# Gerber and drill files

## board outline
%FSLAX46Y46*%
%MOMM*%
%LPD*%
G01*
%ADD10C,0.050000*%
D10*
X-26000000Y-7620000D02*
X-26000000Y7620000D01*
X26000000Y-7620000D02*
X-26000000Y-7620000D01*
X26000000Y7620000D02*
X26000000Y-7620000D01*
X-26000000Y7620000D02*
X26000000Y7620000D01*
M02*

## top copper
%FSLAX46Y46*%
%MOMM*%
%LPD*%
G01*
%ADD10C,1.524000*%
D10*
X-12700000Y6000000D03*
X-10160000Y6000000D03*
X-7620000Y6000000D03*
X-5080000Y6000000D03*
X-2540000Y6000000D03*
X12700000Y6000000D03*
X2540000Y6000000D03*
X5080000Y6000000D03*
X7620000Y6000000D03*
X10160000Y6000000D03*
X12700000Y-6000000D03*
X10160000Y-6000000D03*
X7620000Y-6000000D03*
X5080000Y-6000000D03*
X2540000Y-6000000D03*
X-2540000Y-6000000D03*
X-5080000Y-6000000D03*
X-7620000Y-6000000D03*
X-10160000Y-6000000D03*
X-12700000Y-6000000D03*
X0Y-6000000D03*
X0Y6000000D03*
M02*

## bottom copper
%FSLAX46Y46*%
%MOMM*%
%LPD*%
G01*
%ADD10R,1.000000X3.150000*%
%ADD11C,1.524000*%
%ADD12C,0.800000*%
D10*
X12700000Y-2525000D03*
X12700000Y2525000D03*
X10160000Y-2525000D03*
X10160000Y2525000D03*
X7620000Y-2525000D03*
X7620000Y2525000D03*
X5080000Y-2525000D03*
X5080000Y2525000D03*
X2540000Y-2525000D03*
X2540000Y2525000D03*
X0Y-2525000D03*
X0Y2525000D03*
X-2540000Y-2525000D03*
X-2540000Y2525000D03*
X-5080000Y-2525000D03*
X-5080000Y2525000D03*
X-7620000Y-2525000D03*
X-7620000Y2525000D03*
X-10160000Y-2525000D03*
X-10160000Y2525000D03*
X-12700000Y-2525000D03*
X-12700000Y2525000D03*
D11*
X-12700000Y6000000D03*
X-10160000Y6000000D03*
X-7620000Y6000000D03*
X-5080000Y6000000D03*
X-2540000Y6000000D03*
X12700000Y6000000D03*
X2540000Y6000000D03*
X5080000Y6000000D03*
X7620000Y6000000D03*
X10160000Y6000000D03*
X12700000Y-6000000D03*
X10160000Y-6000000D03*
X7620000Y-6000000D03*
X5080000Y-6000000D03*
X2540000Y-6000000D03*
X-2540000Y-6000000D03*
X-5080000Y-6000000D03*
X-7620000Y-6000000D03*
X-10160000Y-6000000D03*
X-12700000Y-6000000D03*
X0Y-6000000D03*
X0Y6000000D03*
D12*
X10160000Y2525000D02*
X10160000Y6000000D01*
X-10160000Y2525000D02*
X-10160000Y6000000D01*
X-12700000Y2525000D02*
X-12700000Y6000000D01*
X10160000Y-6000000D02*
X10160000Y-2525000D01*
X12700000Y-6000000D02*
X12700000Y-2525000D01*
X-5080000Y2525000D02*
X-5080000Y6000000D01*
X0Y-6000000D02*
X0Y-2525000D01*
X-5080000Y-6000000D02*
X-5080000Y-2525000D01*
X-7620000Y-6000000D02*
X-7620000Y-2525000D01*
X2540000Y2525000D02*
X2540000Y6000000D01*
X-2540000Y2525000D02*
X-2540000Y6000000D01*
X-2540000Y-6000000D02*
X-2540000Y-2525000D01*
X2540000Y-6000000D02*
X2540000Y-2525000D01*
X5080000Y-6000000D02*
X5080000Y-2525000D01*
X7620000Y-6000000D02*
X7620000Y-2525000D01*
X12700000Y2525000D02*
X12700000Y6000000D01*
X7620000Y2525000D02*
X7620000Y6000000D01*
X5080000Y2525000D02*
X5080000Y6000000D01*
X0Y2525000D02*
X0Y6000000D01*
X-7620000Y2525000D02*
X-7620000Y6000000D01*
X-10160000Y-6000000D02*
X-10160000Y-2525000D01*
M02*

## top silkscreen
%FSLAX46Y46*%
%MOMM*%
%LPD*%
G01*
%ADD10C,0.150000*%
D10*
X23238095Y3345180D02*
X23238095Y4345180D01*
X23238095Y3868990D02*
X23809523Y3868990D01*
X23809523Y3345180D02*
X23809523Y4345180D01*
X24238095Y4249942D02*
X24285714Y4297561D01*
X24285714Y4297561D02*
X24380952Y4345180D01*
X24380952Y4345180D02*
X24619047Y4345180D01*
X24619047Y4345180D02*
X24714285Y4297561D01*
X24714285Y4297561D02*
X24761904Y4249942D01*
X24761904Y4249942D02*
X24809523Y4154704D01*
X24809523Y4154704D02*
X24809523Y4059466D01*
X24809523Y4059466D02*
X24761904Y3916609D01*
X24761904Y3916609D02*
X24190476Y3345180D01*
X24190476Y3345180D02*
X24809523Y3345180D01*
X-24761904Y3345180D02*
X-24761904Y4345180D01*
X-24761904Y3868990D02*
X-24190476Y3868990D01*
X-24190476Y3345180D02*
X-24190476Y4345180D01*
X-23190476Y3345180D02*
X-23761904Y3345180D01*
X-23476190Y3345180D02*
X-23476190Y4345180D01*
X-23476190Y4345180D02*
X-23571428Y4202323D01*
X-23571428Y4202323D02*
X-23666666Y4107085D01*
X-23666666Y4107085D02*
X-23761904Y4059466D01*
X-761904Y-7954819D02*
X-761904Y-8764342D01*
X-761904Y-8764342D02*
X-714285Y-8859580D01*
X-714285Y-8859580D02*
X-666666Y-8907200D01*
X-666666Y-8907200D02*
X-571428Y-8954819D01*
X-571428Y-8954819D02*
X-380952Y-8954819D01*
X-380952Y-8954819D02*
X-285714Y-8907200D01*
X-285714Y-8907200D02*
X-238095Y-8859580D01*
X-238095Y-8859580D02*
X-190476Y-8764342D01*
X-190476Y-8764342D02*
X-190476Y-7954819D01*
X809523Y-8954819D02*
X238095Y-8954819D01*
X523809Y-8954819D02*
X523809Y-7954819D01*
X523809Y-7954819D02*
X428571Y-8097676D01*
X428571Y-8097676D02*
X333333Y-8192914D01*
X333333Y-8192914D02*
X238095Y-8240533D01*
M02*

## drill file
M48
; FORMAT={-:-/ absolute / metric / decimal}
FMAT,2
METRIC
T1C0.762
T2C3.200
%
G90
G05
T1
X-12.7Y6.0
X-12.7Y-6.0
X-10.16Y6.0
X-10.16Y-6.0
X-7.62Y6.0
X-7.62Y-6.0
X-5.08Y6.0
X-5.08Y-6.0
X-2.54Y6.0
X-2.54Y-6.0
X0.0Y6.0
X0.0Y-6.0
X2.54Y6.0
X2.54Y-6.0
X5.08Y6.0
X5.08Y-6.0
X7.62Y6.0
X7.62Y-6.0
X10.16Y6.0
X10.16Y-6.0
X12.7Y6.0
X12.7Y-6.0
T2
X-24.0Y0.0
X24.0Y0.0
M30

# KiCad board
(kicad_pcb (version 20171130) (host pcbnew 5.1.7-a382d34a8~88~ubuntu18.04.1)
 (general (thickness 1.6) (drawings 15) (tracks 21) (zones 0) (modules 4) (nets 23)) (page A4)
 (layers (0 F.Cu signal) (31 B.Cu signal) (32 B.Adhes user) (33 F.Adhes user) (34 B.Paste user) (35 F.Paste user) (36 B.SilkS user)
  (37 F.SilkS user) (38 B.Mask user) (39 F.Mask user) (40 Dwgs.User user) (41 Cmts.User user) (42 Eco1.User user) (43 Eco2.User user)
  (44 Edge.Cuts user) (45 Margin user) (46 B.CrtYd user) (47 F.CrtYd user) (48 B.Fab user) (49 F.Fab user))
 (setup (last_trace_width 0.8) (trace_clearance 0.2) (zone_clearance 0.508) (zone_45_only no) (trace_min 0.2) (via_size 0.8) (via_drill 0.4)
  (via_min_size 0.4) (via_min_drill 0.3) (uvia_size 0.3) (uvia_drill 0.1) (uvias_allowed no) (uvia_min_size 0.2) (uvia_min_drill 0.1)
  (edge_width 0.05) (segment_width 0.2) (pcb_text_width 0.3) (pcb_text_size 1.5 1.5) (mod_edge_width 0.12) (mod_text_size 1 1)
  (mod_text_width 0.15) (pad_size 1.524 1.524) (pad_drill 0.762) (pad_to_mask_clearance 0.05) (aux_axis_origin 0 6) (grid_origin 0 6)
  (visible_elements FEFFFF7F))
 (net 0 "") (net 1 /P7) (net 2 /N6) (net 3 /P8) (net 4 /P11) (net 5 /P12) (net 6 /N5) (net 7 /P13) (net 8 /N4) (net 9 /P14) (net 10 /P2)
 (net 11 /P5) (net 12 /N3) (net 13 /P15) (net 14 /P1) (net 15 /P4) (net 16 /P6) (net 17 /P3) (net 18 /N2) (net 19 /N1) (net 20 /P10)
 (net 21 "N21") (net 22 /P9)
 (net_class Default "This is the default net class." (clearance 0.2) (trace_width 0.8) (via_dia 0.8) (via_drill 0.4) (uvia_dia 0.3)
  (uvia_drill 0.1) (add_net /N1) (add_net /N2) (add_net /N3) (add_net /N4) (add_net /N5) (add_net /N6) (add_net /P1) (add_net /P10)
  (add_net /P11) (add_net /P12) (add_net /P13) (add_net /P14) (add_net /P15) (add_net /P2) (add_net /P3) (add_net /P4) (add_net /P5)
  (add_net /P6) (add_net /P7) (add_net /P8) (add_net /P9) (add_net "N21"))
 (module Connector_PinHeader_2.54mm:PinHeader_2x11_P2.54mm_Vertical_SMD (layer B.Cu) (at 0 0 270)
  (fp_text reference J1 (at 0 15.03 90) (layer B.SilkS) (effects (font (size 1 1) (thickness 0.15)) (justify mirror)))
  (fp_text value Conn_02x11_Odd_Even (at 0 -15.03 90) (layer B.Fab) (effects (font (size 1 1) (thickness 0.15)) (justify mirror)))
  (pad 22 smd rect (at 2.525 -12.7 270) (size 3.15 1) (layers B.Cu B.Paste B.Mask) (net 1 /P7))
  (pad 21 smd rect (at -2.525 -12.7 270) (size 3.15 1) (layers B.Cu B.Paste B.Mask) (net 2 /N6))
  (pad 20 smd rect (at 2.525 -10.16 270) (size 3.15 1) (layers B.Cu B.Paste B.Mask) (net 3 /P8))
  (pad 19 smd rect (at -2.525 -10.16 270) (size 3.15 1) (layers B.Cu B.Paste B.Mask) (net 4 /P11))
  (pad 18 smd rect (at 2.525 -7.62 270) (size 3.15 1) (layers B.Cu B.Paste B.Mask) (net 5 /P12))
  (pad 17 smd rect (at -2.525 -7.62 270) (size 3.15 1) (layers B.Cu B.Paste B.Mask) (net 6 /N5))
  (pad 16 smd rect (at 2.525 -5.08 270) (size 3.15 1) (layers B.Cu B.Paste B.Mask) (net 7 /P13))
  (pad 15 smd rect (at -2.525 -5.08 270) (size 3.15 1) (layers B.Cu B.Paste B.Mask) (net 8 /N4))
  (pad 14 smd rect (at 2.525 -2.54 270) (size 3.15 1) (layers B.Cu B.Paste B.Mask) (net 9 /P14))
  (pad 13 smd rect (at -2.525 -2.54 270) (size 3.15 1) (layers B.Cu B.Paste B.Mask) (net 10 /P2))
  (pad 12 smd rect (at 2.525 0 270) (size 3.15 1) (layers B.Cu B.Paste B.Mask) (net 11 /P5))
  (pad 11 smd rect (at -2.525 0 270) (size 3.15 1) (layers B.Cu B.Paste B.Mask) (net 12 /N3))
  (pad 10 smd rect (at 2.525 2.54 270) (size 3.15 1) (layers B.Cu B.Paste B.Mask) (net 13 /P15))
  (pad 9 smd rect (at -2.525 2.54 270) (size 3.15 1) (layers B.Cu B.Paste B.Mask) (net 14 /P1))
  (pad 8 smd rect (at 2.525 5.08 270) (size 3.15 1) (layers B.Cu B.Paste B.Mask) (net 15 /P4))
  (pad 7 smd rect (at -2.525 5.08 270) (size 3.15 1) (layers B.Cu B.Paste B.Mask) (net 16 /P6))
  (pad 6 smd rect (at 2.525 7.62 270) (size 3.15 1) (layers B.Cu B.Paste B.Mask) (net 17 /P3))
  (pad 5 smd rect (at -2.525 7.62 270) (size 3.15 1) (layers B.Cu B.Paste B.Mask) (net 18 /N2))
  (pad 4 smd rect (at 2.525 10.16 270) (size 3.15 1) (layers B.Cu B.Paste B.Mask) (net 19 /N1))
  (pad 3 smd rect (at -2.525 10.16 270) (size 3.15 1) (layers B.Cu B.Paste B.Mask) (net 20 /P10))
  (pad 2 smd rect (at 2.525 12.7 270) (size 3.15 1) (layers B.Cu B.Paste B.Mask) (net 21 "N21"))
  (pad 1 smd rect (at -2.525 12.7 270) (size 3.15 1) (layers B.Cu B.Paste B.Mask) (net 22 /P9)))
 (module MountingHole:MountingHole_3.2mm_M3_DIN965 (layer F.Cu) (at 24 0)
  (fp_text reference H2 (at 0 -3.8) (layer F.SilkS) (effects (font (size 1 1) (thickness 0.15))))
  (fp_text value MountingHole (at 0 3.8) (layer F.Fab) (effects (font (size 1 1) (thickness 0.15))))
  (pad 1 np_thru_hole circle (at 0 0) (size 3.2 3.2) (drill 3.2) (layers *.Cu *.Mask)))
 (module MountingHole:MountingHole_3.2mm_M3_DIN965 (layer F.Cu) (at -24 0)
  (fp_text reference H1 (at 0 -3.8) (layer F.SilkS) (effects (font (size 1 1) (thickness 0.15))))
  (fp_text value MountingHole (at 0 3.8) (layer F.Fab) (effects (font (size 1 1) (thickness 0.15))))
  (pad 1 np_thru_hole circle (at 0 0) (size 3.2 3.2) (drill 3.2) (layers *.Cu *.Mask)))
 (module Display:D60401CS (layer F.Cu) (at 0 0)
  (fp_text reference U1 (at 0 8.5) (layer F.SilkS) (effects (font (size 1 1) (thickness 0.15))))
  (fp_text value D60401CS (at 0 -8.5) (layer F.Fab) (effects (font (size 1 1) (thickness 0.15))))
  (pad 22 thru_hole circle (at -12.7 -6) (size 1.524 1.524) (drill 0.762) (layers *.Cu *.Mask) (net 22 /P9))
  (pad 21 thru_hole circle (at -10.16 -6) (size 1.524 1.524) (drill 0.762) (layers *.Cu *.Mask) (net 20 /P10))
  (pad 20 thru_hole circle (at -7.62 -6) (size 1.524 1.524) (drill 0.762) (layers *.Cu *.Mask) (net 18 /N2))
  (pad 19 thru_hole circle (at -5.08 -6) (size 1.524 1.524) (drill 0.762) (layers *.Cu *.Mask) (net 16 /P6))
  (pad 18 thru_hole circle (at -2.54 -6) (size 1.524 1.524) (drill 0.762) (layers *.Cu *.Mask) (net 14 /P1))
  (pad 12 thru_hole circle (at 12.7 -6) (size 1.524 1.524) (drill 0.762) (layers *.Cu *.Mask) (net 2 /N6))
  (pad 16 thru_hole circle (at 2.54 -6) (size 1.524 1.524) (drill 0.762) (layers *.Cu *.Mask) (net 10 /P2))
  (pad 15 thru_hole circle (at 5.08 -6) (size 1.524 1.524) (drill 0.762) (layers *.Cu *.Mask) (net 8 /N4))
  (pad 14 thru_hole circle (at 7.62 -6) (size 1.524 1.524) (drill 0.762) (layers *.Cu *.Mask) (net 6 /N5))
  (pad 13 thru_hole circle (at 10.16 -6) (size 1.524 1.524) (drill 0.762) (layers *.Cu *.Mask) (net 4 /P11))
  (pad 11 thru_hole circle (at 12.7 6) (size 1.524 1.524) (drill 0.762) (layers *.Cu *.Mask) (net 1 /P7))
  (pad 10 thru_hole circle (at 10.16 6) (size 1.524 1.524) (drill 0.762) (layers *.Cu *.Mask) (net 3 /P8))
  (pad 9 thru_hole circle (at 7.62 6) (size 1.524 1.524) (drill 0.762) (layers *.Cu *.Mask) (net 5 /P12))
  (pad 8 thru_hole circle (at 5.08 6) (size 1.524 1.524) (drill 0.762) (layers *.Cu *.Mask) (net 7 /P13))
  (pad 7 thru_hole circle (at 2.54 6) (size 1.524 1.524) (drill 0.762) (layers *.Cu *.Mask) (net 9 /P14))
  (pad 5 thru_hole circle (at -2.54 6) (size 1.524 1.524) (drill 0.762) (layers *.Cu *.Mask) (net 13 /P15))
  (pad 4 thru_hole circle (at -5.08 6) (size 1.524 1.524) (drill 0.762) (layers *.Cu *.Mask) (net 15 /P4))
  (pad 3 thru_hole circle (at -7.62 6) (size 1.524 1.524) (drill 0.762) (layers *.Cu *.Mask) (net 17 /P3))
  (pad 2 thru_hole circle (at -10.16 6) (size 1.524 1.524) (drill 0.762) (layers *.Cu *.Mask) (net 19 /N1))
  (pad 1 thru_hole circle (at -12.7 6) (size 1.524 1.524) (drill 0.762) (layers *.Cu *.Mask))
  (pad 6 thru_hole circle (at 0 6) (size 1.524 1.524) (drill 0.762) (layers *.Cu *.Mask) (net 11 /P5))
  (pad 17 thru_hole circle (at 0 -6) (size 1.524 1.524) (drill 0.762) (layers *.Cu *.Mask) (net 12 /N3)))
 (gr_line (start -26 7.62) (end -26 -7.62) (layer Edge.Cuts) (width 0.05))
 (gr_line (start 26 7.62) (end -26 7.62) (layer Edge.Cuts) (width 0.05))
 (gr_line (start 26 -7.62) (end 26 7.62) (layer Edge.Cuts) (width 0.05))
 (gr_line (start -26 -7.62) (end 26 -7.62) (layer Edge.Cuts) (width 0.05))
 (segment (start 10.16 -2.525) (end 10.16 -6) (width 0.8) (layer B.Cu) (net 4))
 (segment (start -10.16 -2.525) (end -10.16 -6) (width 0.8) (layer B.Cu) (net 20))
 (segment (start -12.7 -2.525) (end -12.7 -6) (width 0.8) (layer B.Cu) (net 22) (status 30))
 (segment (start 10.16 6) (end 10.16 2.525) (width 0.8) (layer B.Cu) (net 3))
 (segment (start 12.7 6) (end 12.7 2.525) (width 0.8) (layer B.Cu) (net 1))
 (segment (start -5.08 -2.525) (end -5.08 -6) (width 0.8) (layer B.Cu) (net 16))
 (segment (start 0 6) (end 0 2.525) (width 0.8) (layer B.Cu) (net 11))
 (segment (start -5.08 6) (end -5.08 2.525) (width 0.8) (layer B.Cu) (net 15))
 (segment (start -7.62 6) (end -7.62 2.525) (width 0.8) (layer B.Cu) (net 17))
 (segment (start 2.54 -2.525) (end 2.54 -6) (width 0.8) (layer B.Cu) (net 10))
 (segment (start -2.54 -2.525) (end -2.54 -6) (width 0.8) (layer B.Cu) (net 14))
 (segment (start -2.54 6) (end -2.54 2.525) (width 0.8) (layer B.Cu) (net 13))
 (segment (start 2.54 6) (end 2.54 2.525) (width 0.8) (layer B.Cu) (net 9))
 (segment (start 5.08 6) (end 5.08 2.525) (width 0.8) (layer B.Cu) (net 7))
 (segment (start 7.62 6) (end 7.62 2.525) (width 0.8) (layer B.Cu) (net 5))
 (segment (start 12.7 -2.525) (end 12.7 -6) (width 0.8) (layer B.Cu) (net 2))
 (segment (start 7.62 -2.525) (end 7.62 -6) (width 0.8) (layer B.Cu) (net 6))
 (segment (start 5.08 -2.525) (end 5.08 -6) (width 0.8) (layer B.Cu) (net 8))
 (segment (start 0 -2.525) (end 0 -6) (width 0.8) (layer B.Cu) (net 12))
 (segment (start -7.62 -2.525) (end -7.62 -6) (width 0.8) (layer B.Cu) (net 18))
 (segment (start -10.16 6) (end -10.16 2.525) (width 0.8) (layer B.Cu) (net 19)))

